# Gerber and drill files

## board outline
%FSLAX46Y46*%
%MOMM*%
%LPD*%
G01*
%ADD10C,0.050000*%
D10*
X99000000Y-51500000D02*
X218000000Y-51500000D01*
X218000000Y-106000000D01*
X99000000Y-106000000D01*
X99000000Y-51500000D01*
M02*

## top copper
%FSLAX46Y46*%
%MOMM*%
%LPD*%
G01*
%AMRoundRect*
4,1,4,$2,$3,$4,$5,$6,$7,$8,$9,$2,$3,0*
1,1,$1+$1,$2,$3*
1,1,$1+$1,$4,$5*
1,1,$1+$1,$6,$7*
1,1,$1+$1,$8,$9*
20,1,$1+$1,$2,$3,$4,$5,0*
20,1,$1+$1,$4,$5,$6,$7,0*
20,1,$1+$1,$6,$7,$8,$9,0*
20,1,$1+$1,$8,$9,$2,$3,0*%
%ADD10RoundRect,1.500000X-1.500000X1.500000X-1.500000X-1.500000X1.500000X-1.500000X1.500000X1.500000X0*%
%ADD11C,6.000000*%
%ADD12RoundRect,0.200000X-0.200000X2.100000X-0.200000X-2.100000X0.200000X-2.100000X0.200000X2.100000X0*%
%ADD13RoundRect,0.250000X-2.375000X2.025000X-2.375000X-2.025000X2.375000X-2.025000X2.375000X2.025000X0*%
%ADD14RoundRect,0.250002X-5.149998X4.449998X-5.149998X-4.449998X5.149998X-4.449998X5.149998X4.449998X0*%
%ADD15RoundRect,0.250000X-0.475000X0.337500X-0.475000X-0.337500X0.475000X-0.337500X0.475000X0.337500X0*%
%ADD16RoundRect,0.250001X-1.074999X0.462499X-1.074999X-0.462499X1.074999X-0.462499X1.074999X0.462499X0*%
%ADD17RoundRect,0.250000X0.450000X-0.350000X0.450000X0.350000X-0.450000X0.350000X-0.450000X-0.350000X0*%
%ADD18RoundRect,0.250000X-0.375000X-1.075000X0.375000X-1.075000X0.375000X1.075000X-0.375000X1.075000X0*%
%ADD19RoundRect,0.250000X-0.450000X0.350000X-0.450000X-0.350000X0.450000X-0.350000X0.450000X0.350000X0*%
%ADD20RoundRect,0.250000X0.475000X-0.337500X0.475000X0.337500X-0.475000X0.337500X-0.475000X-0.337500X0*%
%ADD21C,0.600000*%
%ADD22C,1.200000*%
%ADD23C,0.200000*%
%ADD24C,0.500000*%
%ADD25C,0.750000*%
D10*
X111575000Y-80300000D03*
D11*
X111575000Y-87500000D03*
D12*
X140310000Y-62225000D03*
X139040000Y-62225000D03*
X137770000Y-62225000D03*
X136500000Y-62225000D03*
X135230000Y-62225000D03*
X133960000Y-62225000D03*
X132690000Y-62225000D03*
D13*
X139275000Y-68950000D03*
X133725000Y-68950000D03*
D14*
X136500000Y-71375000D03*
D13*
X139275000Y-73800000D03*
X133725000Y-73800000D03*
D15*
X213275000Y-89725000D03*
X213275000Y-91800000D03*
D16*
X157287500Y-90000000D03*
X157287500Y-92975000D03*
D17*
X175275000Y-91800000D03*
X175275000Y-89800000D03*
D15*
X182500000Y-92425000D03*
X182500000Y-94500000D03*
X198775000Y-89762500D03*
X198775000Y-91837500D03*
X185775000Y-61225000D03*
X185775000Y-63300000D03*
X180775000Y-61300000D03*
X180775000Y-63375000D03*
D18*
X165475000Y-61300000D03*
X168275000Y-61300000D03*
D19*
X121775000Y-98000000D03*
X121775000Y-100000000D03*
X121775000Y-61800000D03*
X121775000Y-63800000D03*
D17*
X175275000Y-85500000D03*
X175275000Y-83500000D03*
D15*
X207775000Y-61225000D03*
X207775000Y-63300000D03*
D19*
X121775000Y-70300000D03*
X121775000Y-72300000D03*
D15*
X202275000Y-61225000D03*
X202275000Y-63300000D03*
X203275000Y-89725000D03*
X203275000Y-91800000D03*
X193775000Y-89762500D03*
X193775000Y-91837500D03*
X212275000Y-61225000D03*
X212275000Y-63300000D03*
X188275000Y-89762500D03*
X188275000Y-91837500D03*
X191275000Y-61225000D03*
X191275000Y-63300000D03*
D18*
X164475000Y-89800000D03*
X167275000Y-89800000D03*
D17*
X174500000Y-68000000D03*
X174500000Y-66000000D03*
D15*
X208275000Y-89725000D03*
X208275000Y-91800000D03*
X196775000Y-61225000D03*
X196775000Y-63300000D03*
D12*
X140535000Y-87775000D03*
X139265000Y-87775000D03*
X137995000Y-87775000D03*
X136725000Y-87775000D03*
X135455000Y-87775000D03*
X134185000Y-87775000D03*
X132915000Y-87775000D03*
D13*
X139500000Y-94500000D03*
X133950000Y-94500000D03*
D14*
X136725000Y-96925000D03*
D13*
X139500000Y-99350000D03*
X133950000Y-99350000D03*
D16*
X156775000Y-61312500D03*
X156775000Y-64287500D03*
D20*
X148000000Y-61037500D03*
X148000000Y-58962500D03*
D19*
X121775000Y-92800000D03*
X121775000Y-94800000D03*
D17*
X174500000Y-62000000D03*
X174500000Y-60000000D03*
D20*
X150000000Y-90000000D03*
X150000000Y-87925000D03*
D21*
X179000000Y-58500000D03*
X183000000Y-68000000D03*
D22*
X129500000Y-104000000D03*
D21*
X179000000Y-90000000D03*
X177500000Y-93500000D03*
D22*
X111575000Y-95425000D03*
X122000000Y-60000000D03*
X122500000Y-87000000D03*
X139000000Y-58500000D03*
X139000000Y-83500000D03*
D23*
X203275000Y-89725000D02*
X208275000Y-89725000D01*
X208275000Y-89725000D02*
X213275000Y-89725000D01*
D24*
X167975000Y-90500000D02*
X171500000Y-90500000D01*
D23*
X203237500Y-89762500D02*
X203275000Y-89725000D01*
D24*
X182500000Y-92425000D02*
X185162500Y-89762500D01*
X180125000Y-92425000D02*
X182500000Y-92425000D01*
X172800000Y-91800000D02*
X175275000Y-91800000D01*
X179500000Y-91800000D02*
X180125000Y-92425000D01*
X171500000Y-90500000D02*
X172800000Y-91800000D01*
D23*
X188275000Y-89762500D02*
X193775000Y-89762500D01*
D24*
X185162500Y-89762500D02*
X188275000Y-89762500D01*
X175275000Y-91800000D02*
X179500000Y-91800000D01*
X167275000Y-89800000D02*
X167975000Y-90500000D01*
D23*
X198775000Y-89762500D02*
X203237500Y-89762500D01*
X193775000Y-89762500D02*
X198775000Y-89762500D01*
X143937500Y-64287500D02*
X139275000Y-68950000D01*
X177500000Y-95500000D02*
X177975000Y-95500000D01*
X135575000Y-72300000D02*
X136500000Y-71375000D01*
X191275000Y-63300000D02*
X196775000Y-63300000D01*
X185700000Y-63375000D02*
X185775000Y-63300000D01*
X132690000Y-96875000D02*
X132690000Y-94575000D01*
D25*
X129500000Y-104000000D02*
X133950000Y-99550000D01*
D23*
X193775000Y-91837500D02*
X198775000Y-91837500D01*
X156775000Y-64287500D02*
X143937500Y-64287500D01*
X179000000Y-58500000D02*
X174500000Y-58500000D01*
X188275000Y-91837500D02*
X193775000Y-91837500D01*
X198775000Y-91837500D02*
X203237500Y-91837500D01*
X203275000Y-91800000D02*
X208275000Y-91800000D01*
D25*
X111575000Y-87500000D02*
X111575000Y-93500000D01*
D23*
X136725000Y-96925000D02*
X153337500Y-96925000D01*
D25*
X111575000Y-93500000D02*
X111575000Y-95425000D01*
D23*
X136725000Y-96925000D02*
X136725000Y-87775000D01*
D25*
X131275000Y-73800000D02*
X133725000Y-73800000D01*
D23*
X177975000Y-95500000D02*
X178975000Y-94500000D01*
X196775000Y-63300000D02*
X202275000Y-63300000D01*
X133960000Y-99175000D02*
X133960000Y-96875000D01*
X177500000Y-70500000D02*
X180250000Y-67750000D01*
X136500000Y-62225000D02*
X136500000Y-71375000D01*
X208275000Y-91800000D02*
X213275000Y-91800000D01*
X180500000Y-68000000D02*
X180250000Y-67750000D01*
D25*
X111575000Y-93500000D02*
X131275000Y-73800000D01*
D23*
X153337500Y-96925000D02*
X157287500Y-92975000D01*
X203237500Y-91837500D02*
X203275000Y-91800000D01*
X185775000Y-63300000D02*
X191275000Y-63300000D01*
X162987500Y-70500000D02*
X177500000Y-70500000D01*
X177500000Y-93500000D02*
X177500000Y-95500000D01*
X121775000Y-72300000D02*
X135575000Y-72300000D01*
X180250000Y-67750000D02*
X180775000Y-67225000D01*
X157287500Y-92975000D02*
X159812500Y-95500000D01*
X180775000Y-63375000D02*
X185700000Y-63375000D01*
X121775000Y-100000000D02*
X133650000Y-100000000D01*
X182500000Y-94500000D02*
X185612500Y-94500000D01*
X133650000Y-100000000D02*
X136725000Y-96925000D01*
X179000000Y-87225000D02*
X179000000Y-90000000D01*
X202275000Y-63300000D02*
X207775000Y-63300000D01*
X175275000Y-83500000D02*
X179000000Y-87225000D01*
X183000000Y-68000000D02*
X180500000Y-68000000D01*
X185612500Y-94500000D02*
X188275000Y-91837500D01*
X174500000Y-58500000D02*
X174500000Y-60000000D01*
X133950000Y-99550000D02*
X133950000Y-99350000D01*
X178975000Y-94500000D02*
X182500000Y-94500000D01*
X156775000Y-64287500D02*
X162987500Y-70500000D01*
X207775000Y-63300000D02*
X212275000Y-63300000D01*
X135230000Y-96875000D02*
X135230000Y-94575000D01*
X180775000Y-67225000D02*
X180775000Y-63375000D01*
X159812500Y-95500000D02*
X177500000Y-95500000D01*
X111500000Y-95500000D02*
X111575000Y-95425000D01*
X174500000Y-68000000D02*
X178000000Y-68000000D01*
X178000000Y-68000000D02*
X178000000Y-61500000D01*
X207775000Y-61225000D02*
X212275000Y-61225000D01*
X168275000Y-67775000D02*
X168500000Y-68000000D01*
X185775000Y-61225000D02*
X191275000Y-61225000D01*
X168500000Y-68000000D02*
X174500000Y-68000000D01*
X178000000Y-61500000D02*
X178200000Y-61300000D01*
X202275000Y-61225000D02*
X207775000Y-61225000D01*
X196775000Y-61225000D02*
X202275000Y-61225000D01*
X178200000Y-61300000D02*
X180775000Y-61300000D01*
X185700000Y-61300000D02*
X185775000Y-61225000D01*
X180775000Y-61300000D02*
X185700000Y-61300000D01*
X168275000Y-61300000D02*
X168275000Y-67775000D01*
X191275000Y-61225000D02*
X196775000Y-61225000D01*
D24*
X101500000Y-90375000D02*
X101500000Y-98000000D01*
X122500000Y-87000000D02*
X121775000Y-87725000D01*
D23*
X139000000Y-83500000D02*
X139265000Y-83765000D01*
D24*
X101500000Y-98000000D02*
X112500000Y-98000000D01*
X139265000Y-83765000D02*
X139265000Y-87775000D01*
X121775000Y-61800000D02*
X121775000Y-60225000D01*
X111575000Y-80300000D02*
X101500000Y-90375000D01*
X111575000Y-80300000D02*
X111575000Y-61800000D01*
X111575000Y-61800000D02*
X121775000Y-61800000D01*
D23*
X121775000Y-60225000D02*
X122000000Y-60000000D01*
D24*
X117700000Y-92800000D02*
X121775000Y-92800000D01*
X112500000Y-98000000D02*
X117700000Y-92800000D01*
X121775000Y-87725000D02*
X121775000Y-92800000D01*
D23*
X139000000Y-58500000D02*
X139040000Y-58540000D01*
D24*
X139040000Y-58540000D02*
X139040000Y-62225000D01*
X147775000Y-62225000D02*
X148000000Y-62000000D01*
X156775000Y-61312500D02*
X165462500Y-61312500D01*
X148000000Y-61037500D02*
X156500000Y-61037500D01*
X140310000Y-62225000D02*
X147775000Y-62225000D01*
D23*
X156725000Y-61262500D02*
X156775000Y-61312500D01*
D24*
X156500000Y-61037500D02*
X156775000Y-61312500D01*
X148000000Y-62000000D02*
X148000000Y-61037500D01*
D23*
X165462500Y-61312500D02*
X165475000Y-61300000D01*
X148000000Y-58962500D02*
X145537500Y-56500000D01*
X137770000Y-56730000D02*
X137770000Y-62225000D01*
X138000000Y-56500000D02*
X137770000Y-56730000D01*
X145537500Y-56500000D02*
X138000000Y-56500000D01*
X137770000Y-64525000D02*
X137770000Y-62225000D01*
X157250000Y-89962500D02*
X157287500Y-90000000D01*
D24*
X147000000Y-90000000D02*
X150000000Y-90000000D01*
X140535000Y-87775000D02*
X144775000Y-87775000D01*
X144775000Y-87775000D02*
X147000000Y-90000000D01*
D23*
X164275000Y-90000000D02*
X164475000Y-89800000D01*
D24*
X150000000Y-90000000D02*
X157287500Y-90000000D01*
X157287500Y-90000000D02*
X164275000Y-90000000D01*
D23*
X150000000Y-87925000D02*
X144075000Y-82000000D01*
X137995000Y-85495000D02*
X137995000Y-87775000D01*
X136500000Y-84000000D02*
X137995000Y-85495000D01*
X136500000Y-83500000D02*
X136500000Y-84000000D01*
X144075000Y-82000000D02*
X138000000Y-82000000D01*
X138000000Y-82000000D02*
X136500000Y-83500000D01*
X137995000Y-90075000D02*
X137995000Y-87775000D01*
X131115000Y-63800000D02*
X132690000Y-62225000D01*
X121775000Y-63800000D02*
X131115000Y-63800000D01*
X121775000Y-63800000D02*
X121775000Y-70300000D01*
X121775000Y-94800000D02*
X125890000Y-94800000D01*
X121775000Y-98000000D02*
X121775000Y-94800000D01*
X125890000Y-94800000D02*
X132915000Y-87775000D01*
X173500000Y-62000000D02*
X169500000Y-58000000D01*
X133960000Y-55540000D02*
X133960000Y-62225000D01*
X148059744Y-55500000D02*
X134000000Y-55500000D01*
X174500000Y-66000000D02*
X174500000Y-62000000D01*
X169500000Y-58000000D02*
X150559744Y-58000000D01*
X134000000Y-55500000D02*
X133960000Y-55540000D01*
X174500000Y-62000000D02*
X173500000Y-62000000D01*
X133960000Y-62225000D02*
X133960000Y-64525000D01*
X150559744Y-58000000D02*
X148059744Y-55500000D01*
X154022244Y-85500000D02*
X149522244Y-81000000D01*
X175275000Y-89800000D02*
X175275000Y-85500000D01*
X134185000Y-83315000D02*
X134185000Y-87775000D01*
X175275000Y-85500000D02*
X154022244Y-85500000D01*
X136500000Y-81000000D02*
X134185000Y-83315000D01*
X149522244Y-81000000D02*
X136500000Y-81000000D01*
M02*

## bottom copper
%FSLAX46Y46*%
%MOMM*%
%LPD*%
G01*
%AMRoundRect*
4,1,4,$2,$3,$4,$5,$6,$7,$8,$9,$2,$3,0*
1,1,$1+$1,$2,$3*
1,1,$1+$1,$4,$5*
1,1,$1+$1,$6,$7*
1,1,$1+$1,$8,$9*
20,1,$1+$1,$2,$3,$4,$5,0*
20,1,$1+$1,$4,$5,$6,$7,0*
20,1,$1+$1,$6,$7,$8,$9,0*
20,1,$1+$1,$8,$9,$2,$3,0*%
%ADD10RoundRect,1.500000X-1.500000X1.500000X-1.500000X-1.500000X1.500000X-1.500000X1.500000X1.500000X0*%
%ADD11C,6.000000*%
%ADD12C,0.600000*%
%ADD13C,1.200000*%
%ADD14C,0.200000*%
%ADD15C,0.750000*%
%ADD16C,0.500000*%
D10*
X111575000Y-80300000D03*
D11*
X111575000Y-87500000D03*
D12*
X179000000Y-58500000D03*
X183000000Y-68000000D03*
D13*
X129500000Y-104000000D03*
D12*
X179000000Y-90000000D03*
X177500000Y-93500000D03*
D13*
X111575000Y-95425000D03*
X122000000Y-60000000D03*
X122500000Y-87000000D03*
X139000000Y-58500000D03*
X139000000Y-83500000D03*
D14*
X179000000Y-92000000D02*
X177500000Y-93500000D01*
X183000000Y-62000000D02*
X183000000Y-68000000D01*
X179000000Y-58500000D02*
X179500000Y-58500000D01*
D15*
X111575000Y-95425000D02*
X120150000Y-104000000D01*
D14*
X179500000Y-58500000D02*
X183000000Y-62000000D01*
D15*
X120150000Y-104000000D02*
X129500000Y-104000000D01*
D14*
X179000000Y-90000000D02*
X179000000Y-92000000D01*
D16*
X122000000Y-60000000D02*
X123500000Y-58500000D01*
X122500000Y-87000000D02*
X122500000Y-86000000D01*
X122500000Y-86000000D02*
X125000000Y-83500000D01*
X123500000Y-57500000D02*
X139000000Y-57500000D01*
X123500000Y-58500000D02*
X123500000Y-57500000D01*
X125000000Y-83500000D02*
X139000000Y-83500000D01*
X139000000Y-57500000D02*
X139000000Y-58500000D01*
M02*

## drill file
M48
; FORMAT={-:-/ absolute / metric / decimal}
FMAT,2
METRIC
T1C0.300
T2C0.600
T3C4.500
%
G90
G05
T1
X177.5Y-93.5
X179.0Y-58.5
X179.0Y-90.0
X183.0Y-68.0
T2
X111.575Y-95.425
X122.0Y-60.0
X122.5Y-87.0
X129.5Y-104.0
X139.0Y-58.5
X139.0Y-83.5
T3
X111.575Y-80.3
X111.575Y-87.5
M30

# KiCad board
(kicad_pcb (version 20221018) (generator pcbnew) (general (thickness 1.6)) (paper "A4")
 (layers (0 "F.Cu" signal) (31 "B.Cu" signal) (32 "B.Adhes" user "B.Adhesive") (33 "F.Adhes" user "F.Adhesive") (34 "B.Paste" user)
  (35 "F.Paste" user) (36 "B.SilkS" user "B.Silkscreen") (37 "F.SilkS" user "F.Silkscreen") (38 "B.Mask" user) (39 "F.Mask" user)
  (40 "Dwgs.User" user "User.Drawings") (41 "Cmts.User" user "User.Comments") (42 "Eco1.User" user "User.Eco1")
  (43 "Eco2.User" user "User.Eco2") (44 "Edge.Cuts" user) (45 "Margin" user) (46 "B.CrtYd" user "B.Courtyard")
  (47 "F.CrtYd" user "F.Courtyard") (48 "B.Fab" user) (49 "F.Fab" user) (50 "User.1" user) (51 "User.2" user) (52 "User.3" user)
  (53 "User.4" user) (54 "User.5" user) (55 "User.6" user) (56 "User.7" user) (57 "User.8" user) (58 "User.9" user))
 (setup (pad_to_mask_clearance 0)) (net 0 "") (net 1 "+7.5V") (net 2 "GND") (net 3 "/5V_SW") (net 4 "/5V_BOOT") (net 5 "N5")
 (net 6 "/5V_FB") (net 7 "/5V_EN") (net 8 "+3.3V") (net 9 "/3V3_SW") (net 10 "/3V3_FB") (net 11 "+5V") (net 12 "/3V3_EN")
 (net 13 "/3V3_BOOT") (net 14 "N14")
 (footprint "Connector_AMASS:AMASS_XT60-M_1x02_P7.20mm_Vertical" (layer "F.Cu") (at 111.575 80.3 -90)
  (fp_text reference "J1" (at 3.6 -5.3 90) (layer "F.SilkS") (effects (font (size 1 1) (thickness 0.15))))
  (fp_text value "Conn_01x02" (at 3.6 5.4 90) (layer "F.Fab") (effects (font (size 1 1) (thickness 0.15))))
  (pad "1" thru_hole roundrect (at 0 0 270) (size 6 6) (drill 4.5) (layers "*.Cu" "*.Mask") (roundrect_rratio 0.25) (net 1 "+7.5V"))
  (pad "2" thru_hole circle (at 7.2 0 270) (size 6 6) (drill 4.5) (layers "*.Cu" "*.Mask") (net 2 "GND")))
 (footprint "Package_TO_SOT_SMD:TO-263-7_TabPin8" (layer "F.Cu") (at 136.5 69.875 -90)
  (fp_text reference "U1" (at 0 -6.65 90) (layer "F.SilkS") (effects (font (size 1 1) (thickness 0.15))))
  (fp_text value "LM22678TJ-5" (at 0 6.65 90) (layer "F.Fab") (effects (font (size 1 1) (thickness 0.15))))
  (pad "1" smd roundrect (at -7.65 -3.81 270) (size 4.6 0.8) (layers "F.Cu" "F.Paste" "F.Mask") (roundrect_rratio 0.25) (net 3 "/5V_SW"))
  (pad "2" smd roundrect (at -7.65 -2.54 270) (size 4.6 0.8) (layers "F.Cu" "F.Paste" "F.Mask") (roundrect_rratio 0.25) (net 1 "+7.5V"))
  (pad "3" smd roundrect (at -7.65 -1.27 270) (size 4.6 0.8) (layers "F.Cu" "F.Paste" "F.Mask") (roundrect_rratio 0.25) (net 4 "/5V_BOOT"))
  (pad "4" smd roundrect (at -7.65 0 270) (size 4.6 0.8) (layers "F.Cu" "F.Paste" "F.Mask") (roundrect_rratio 0.25) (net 2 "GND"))
  (pad "5" smd roundrect (at -7.65 1.27 270) (size 4.6 0.8) (layers "F.Cu" "F.Paste" "F.Mask") (roundrect_rratio 0.25) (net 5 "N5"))
  (pad "6" smd roundrect (at -7.65 2.54 270) (size 4.6 0.8) (layers "F.Cu" "F.Paste" "F.Mask") (roundrect_rratio 0.25) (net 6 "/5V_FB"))
  (pad "7" smd roundrect (at -7.65 3.81 270) (size 4.6 0.8) (layers "F.Cu" "F.Paste" "F.Mask") (roundrect_rratio 0.25) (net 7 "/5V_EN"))
  (pad "8" smd roundrect (at -0.925 -2.775 270) (size 4.55 5.25) (layers "F.Cu" "F.Paste") (roundrect_rratio 0.054945) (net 2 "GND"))
  (pad "8" smd roundrect (at -0.925 2.775 270) (size 4.55 5.25) (layers "F.Cu" "F.Paste") (roundrect_rratio 0.054945) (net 2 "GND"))
  (pad "8" smd roundrect (at 1.5 0 270) (size 9.4 10.8) (layers "F.Cu" "F.Mask") (roundrect_rratio 0.026596) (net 2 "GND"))
  (pad "8" smd roundrect (at 3.925 -2.775 270) (size 4.55 5.25) (layers "F.Cu" "F.Paste") (roundrect_rratio 0.054945) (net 2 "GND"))
  (pad "8" smd roundrect (at 3.925 2.775 270) (size 4.55 5.25) (layers "F.Cu" "F.Paste") (roundrect_rratio 0.054945) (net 2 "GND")))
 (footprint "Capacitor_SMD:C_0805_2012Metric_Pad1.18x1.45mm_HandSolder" (layer "F.Cu") (at 213.275 90.7625 -90)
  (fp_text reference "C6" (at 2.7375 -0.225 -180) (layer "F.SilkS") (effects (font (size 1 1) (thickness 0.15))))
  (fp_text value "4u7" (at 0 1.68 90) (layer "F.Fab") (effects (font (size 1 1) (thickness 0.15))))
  (pad "1" smd roundrect (at -1.0375 0 270) (size 1.175 1.45) (layers "F.Cu" "F.Paste" "F.Mask") (roundrect_rratio 0.212766) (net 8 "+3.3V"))
  (pad "2" smd roundrect (at 1.0375 0 270) (size 1.175 1.45) (layers "F.Cu" "F.Paste" "F.Mask") (roundrect_rratio 0.212766) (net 2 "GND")))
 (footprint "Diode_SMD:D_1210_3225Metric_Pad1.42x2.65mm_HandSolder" (layer "F.Cu") (at 157.2875 91.4875 -90)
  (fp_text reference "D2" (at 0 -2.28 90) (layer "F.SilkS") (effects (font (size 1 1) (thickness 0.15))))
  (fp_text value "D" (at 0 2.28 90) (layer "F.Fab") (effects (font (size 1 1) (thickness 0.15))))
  (pad "1" smd roundrect (at -1.4875 0 270) (size 1.425 2.65) (layers "F.Cu" "F.Paste" "F.Mask") (roundrect_rratio 0.175439)
   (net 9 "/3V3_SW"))
  (pad "2" smd roundrect (at 1.4875 0 270) (size 1.425 2.65) (layers "F.Cu" "F.Paste" "F.Mask") (roundrect_rratio 0.175439) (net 2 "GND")))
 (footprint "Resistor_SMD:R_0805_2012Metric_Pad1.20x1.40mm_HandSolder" (layer "F.Cu") (at 175.275 90.8 90)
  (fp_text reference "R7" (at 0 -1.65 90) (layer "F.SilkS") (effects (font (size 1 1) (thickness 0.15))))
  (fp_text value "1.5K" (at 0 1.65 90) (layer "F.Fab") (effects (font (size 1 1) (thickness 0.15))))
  (pad "1" smd roundrect (at -1 0 90) (size 1.2 1.4) (layers "F.Cu" "F.Paste" "F.Mask") (roundrect_rratio 0.208333) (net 8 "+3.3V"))
  (pad "2" smd roundrect (at 1 0 90) (size 1.2 1.4) (layers "F.Cu" "F.Paste" "F.Mask") (roundrect_rratio 0.208333) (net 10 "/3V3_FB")))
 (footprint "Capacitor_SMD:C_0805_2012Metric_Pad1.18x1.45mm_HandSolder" (layer "F.Cu") (at 182.5 93.4625 -90)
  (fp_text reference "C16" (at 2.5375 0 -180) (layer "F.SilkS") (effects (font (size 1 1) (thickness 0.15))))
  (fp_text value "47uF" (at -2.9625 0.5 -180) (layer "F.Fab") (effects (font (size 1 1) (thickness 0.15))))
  (pad "1" smd roundrect (at -1.0375 0 270) (size 1.175 1.45) (layers "F.Cu" "F.Paste" "F.Mask") (roundrect_rratio 0.212766) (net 8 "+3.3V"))
  (pad "2" smd roundrect (at 1.0375 0 270) (size 1.175 1.45) (layers "F.Cu" "F.Paste" "F.Mask") (roundrect_rratio 0.212766) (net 2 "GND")))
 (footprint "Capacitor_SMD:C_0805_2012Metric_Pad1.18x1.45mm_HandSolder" (layer "F.Cu") (at 198.775 90.8 -90)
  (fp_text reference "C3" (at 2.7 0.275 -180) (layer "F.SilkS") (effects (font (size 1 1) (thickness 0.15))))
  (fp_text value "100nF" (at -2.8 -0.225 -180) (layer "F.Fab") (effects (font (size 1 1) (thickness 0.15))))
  (pad "1" smd roundrect (at -1.0375 0 270) (size 1.175 1.45) (layers "F.Cu" "F.Paste" "F.Mask") (roundrect_rratio 0.212766) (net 8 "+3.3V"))
  (pad "2" smd roundrect (at 1.0375 0 270) (size 1.175 1.45) (layers "F.Cu" "F.Paste" "F.Mask") (roundrect_rratio 0.212766) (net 2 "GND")))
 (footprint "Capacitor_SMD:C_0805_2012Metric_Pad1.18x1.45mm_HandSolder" (layer "F.Cu") (at 185.775 62.2625 -90)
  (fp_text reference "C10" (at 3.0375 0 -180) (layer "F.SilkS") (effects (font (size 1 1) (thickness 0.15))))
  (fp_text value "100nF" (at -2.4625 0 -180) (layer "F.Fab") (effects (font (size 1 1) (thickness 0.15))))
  (pad "1" smd roundrect (at -1.0375 0 270) (size 1.175 1.45) (layers "F.Cu" "F.Paste" "F.Mask") (roundrect_rratio 0.212766) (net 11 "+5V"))
  (pad "2" smd roundrect (at 1.0375 0 270) (size 1.175 1.45) (layers "F.Cu" "F.Paste" "F.Mask") (roundrect_rratio 0.212766) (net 2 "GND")))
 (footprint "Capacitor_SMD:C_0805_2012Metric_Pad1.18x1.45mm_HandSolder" (layer "F.Cu") (at 180.775 62.3375 -90)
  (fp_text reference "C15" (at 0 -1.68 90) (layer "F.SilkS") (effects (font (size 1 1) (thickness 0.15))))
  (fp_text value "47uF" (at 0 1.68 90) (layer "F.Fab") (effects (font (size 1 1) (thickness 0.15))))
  (pad "1" smd roundrect (at -1.0375 0 270) (size 1.175 1.45) (layers "F.Cu" "F.Paste" "F.Mask") (roundrect_rratio 0.212766) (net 11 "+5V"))
  (pad "2" smd roundrect (at 1.0375 0 270) (size 1.175 1.45) (layers "F.Cu" "F.Paste" "F.Mask") (roundrect_rratio 0.212766) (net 2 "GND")))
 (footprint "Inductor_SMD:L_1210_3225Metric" (layer "F.Cu") (at 166.875 61.3)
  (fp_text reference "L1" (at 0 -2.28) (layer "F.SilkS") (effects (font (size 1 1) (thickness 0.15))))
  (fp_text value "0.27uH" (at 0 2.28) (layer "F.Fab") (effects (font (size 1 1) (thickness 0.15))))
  (pad "1" smd roundrect (at -1.4 0) (size 1.25 2.65) (layers "F.Cu" "F.Paste" "F.Mask") (roundrect_rratio 0.2) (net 3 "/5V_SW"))
  (pad "2" smd roundrect (at 1.4 0) (size 1.25 2.65) (layers "F.Cu" "F.Paste" "F.Mask") (roundrect_rratio 0.2) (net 11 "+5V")))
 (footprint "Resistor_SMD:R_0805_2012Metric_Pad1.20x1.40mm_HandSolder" (layer "F.Cu") (at 121.775 99 -90)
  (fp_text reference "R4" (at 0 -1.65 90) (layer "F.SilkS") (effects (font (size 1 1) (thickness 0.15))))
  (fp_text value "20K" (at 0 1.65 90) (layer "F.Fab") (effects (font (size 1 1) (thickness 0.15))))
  (pad "1" smd roundrect (at -1 0 270) (size 1.2 1.4) (layers "F.Cu" "F.Paste" "F.Mask") (roundrect_rratio 0.208333) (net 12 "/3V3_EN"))
  (pad "2" smd roundrect (at 1 0 270) (size 1.2 1.4) (layers "F.Cu" "F.Paste" "F.Mask") (roundrect_rratio 0.208333) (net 2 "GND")))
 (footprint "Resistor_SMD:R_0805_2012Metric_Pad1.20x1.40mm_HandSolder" (layer "F.Cu") (at 121.775 62.8 -90)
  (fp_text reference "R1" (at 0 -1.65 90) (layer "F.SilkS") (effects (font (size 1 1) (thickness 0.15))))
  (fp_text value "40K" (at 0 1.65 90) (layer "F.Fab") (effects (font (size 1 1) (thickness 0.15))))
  (pad "1" smd roundrect (at -1 0 270) (size 1.2 1.4) (layers "F.Cu" "F.Paste" "F.Mask") (roundrect_rratio 0.208333) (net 1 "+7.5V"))
  (pad "2" smd roundrect (at 1 0 270) (size 1.2 1.4) (layers "F.Cu" "F.Paste" "F.Mask") (roundrect_rratio 0.208333) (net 7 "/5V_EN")))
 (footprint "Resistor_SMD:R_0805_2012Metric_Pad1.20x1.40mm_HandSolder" (layer "F.Cu") (at 175.275 84.5 90)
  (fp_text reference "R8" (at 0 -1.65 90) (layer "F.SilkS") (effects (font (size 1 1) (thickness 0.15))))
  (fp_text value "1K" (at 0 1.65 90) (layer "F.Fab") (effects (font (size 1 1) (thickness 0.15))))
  (pad "1" smd roundrect (at -1 0 90) (size 1.2 1.4) (layers "F.Cu" "F.Paste" "F.Mask") (roundrect_rratio 0.208333) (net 10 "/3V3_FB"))
  (pad "2" smd roundrect (at 1 0 90) (size 1.2 1.4) (layers "F.Cu" "F.Paste" "F.Mask") (roundrect_rratio 0.208333) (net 2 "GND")))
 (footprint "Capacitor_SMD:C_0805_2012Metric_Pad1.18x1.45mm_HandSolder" (layer "F.Cu") (at 207.775 62.2625 -90)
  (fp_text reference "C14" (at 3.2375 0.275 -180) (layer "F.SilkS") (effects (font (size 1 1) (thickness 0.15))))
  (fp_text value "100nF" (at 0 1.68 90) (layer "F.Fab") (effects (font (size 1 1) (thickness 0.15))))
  (pad "1" smd roundrect (at -1.0375 0 270) (size 1.175 1.45) (layers "F.Cu" "F.Paste" "F.Mask") (roundrect_rratio 0.212766) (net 11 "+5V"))
  (pad "2" smd roundrect (at 1.0375 0 270) (size 1.175 1.45) (layers "F.Cu" "F.Paste" "F.Mask") (roundrect_rratio 0.212766) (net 2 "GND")))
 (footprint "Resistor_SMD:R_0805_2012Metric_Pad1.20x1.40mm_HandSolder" (layer "F.Cu") (at 121.775 71.3 -90)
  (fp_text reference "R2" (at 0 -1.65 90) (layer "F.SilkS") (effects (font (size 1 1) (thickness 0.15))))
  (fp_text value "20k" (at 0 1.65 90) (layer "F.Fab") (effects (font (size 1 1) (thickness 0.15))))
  (pad "1" smd roundrect (at -1 0 270) (size 1.2 1.4) (layers "F.Cu" "F.Paste" "F.Mask") (roundrect_rratio 0.208333) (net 7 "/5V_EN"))
  (pad "2" smd roundrect (at 1 0 270) (size 1.2 1.4) (layers "F.Cu" "F.Paste" "F.Mask") (roundrect_rratio 0.208333) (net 2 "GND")))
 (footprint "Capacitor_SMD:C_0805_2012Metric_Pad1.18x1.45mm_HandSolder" (layer "F.Cu") (at 202.275 62.2625 -90)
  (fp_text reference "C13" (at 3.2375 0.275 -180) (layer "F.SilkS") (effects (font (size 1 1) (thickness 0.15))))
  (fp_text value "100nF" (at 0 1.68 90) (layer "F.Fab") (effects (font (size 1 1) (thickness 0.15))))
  (pad "1" smd roundrect (at -1.0375 0 270) (size 1.175 1.45) (layers "F.Cu" "F.Paste" "F.Mask") (roundrect_rratio 0.212766) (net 11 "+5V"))
  (pad "2" smd roundrect (at 1.0375 0 270) (size 1.175 1.45) (layers "F.Cu" "F.Paste" "F.Mask") (roundrect_rratio 0.212766) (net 2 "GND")))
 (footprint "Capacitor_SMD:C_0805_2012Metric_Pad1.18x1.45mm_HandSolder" (layer "F.Cu") (at 203.275 90.7625 -90)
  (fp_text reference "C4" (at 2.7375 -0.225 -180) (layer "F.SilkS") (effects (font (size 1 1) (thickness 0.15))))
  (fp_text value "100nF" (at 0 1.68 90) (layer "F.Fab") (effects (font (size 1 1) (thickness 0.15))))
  (pad "1" smd roundrect (at -1.0375 0 270) (size 1.175 1.45) (layers "F.Cu" "F.Paste" "F.Mask") (roundrect_rratio 0.212766) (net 8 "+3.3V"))
  (pad "2" smd roundrect (at 1.0375 0 270) (size 1.175 1.45) (layers "F.Cu" "F.Paste" "F.Mask") (roundrect_rratio 0.212766) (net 2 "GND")))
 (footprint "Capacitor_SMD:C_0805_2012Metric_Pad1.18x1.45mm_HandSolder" (layer "F.Cu") (at 193.775 90.8 -90)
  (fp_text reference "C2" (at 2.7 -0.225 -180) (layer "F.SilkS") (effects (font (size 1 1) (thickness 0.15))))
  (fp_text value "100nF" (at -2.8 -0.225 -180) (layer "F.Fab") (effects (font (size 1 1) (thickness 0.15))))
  (pad "1" smd roundrect (at -1.0375 0 270) (size 1.175 1.45) (layers "F.Cu" "F.Paste" "F.Mask") (roundrect_rratio 0.212766) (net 8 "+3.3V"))
  (pad "2" smd roundrect (at 1.0375 0 270) (size 1.175 1.45) (layers "F.Cu" "F.Paste" "F.Mask") (roundrect_rratio 0.212766) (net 2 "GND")))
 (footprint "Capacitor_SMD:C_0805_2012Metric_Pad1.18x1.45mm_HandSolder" (layer "F.Cu") (at 212.275 62.2625 -90)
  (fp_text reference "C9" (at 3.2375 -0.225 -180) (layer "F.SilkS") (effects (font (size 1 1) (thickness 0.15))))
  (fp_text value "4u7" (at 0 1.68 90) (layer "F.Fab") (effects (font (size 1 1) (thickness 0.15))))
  (pad "1" smd roundrect (at -1.0375 0 270) (size 1.175 1.45) (layers "F.Cu" "F.Paste" "F.Mask") (roundrect_rratio 0.212766) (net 11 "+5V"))
  (pad "2" smd roundrect (at 1.0375 0 270) (size 1.175 1.45) (layers "F.Cu" "F.Paste" "F.Mask") (roundrect_rratio 0.212766) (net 2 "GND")))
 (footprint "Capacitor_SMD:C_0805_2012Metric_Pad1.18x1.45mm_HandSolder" (layer "F.Cu") (at 188.275 90.8 -90)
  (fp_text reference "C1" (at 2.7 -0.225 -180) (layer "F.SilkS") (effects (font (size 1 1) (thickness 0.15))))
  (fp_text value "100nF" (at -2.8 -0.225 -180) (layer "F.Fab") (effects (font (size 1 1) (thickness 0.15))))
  (pad "1" smd roundrect (at -1.0375 0 270) (size 1.175 1.45) (layers "F.Cu" "F.Paste" "F.Mask") (roundrect_rratio 0.212766) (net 8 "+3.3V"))
  (pad "2" smd roundrect (at 1.0375 0 270) (size 1.175 1.45) (layers "F.Cu" "F.Paste" "F.Mask") (roundrect_rratio 0.212766) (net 2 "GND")))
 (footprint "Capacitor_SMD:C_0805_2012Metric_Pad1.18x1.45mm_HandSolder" (layer "F.Cu") (at 191.275 62.2625 -90)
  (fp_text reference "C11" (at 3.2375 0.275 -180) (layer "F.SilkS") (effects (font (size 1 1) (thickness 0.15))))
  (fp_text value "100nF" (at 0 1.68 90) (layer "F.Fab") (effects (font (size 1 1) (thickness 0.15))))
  (pad "1" smd roundrect (at -1.0375 0 270) (size 1.175 1.45) (layers "F.Cu" "F.Paste" "F.Mask") (roundrect_rratio 0.212766) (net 11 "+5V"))
  (pad "2" smd roundrect (at 1.0375 0 270) (size 1.175 1.45) (layers "F.Cu" "F.Paste" "F.Mask") (roundrect_rratio 0.212766) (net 2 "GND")))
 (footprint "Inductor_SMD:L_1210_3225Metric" (layer "F.Cu") (at 165.875 89.8)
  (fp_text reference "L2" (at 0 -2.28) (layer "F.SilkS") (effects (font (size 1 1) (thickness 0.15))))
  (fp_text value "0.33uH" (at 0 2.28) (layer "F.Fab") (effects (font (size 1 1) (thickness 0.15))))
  (pad "1" smd roundrect (at -1.4 0) (size 1.25 2.65) (layers "F.Cu" "F.Paste" "F.Mask") (roundrect_rratio 0.2) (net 9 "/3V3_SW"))
  (pad "2" smd roundrect (at 1.4 0) (size 1.25 2.65) (layers "F.Cu" "F.Paste" "F.Mask") (roundrect_rratio 0.2) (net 8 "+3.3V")))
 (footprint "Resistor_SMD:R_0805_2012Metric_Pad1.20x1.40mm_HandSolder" (layer "F.Cu") (at 174.5 67 90)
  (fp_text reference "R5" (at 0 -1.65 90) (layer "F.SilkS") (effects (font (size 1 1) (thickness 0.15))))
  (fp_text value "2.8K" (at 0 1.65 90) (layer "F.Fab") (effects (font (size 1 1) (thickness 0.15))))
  (pad "1" smd roundrect (at -1 0 90) (size 1.2 1.4) (layers "F.Cu" "F.Paste" "F.Mask") (roundrect_rratio 0.208333) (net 11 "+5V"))
  (pad "2" smd roundrect (at 1 0 90) (size 1.2 1.4) (layers "F.Cu" "F.Paste" "F.Mask") (roundrect_rratio 0.208333) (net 6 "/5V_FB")))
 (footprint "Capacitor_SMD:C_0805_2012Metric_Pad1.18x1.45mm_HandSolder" (layer "F.Cu") (at 208.275 90.7625 -90)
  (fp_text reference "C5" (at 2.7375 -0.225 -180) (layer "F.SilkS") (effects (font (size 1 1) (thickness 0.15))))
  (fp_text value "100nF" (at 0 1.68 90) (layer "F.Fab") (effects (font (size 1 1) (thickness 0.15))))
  (pad "1" smd roundrect (at -1.0375 0 270) (size 1.175 1.45) (layers "F.Cu" "F.Paste" "F.Mask") (roundrect_rratio 0.212766) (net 8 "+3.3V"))
  (pad "2" smd roundrect (at 1.0375 0 270) (size 1.175 1.45) (layers "F.Cu" "F.Paste" "F.Mask") (roundrect_rratio 0.212766) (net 2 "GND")))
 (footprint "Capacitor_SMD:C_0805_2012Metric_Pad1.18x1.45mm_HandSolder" (layer "F.Cu") (at 196.775 62.2625 -90)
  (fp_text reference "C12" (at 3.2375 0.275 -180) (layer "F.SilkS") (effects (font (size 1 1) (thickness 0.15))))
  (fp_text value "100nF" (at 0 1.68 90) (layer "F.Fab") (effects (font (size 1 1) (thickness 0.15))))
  (pad "1" smd roundrect (at -1.0375 0 270) (size 1.175 1.45) (layers "F.Cu" "F.Paste" "F.Mask") (roundrect_rratio 0.212766) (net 11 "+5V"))
  (pad "2" smd roundrect (at 1.0375 0 270) (size 1.175 1.45) (layers "F.Cu" "F.Paste" "F.Mask") (roundrect_rratio 0.212766) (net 2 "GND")))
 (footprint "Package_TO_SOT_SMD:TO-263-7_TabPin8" (layer "F.Cu") (at 136.725 95.425 -90)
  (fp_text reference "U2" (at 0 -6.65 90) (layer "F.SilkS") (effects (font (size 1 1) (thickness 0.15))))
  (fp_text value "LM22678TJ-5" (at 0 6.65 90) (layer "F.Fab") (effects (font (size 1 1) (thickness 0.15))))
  (pad "1" smd roundrect (at -7.65 -3.81 270) (size 4.6 0.8) (layers "F.Cu" "F.Paste" "F.Mask") (roundrect_rratio 0.25) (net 9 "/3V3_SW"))
  (pad "2" smd roundrect (at -7.65 -2.54 270) (size 4.6 0.8) (layers "F.Cu" "F.Paste" "F.Mask") (roundrect_rratio 0.25) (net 1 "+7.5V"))
  (pad "3" smd roundrect (at -7.65 -1.27 270) (size 4.6 0.8) (layers "F.Cu" "F.Paste" "F.Mask") (roundrect_rratio 0.25) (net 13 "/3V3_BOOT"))
  (pad "4" smd roundrect (at -7.65 0 270) (size 4.6 0.8) (layers "F.Cu" "F.Paste" "F.Mask") (roundrect_rratio 0.25) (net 2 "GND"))
  (pad "5" smd roundrect (at -7.65 1.27 270) (size 4.6 0.8) (layers "F.Cu" "F.Paste" "F.Mask") (roundrect_rratio 0.25) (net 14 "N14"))
  (pad "6" smd roundrect (at -7.65 2.54 270) (size 4.6 0.8) (layers "F.Cu" "F.Paste" "F.Mask") (roundrect_rratio 0.25) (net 10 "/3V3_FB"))
  (pad "7" smd roundrect (at -7.65 3.81 270) (size 4.6 0.8) (layers "F.Cu" "F.Paste" "F.Mask") (roundrect_rratio 0.25) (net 12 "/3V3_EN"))
  (pad "8" smd roundrect (at -0.925 -2.775 270) (size 4.55 5.25) (layers "F.Cu" "F.Paste") (roundrect_rratio 0.054945) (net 2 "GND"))
  (pad "8" smd roundrect (at -0.925 2.775 270) (size 4.55 5.25) (layers "F.Cu" "F.Paste") (roundrect_rratio 0.054945) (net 2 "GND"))
  (pad "8" smd roundrect (at 1.5 0 270) (size 9.4 10.8) (layers "F.Cu" "F.Mask") (roundrect_rratio 0.026596) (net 2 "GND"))
  (pad "8" smd roundrect (at 3.925 -2.775 270) (size 4.55 5.25) (layers "F.Cu" "F.Paste") (roundrect_rratio 0.054945) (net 2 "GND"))
  (pad "8" smd roundrect (at 3.925 2.775 270) (size 4.55 5.25) (layers "F.Cu" "F.Paste") (roundrect_rratio 0.054945) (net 2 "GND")))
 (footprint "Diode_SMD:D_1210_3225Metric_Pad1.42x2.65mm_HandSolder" (layer "F.Cu") (at 156.775 62.8 -90)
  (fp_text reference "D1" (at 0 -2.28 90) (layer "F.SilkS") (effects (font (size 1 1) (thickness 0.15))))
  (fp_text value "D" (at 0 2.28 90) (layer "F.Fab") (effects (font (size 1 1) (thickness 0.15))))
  (pad "1" smd roundrect (at -1.4875 0 270) (size 1.425 2.65) (layers "F.Cu" "F.Paste" "F.Mask") (roundrect_rratio 0.175439)
   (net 3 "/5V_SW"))
  (pad "2" smd roundrect (at 1.4875 0 270) (size 1.425 2.65) (layers "F.Cu" "F.Paste" "F.Mask") (roundrect_rratio 0.175439) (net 2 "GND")))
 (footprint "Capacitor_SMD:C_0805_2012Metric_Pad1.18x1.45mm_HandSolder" (layer "F.Cu") (at 148 60 90)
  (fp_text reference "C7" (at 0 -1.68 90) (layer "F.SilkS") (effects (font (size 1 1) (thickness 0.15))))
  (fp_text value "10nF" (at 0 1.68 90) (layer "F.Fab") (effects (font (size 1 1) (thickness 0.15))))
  (pad "1" smd roundrect (at -1.0375 0 90) (size 1.175 1.45) (layers "F.Cu" "F.Paste" "F.Mask") (roundrect_rratio 0.212766) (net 3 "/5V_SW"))
  (pad "2" smd roundrect (at 1.0375 0 90) (size 1.175 1.45) (layers "F.Cu" "F.Paste" "F.Mask") (roundrect_rratio 0.212766)
   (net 4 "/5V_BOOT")))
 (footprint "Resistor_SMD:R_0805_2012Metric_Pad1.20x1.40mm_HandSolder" (layer "F.Cu") (at 121.775 93.8 -90)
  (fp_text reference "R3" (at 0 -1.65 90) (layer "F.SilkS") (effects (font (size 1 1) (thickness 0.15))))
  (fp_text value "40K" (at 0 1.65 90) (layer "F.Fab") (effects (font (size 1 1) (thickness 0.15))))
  (pad "1" smd roundrect (at -1 0 270) (size 1.2 1.4) (layers "F.Cu" "F.Paste" "F.Mask") (roundrect_rratio 0.208333) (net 1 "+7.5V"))
  (pad "2" smd roundrect (at 1 0 270) (size 1.2 1.4) (layers "F.Cu" "F.Paste" "F.Mask") (roundrect_rratio 0.208333) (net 12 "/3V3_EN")))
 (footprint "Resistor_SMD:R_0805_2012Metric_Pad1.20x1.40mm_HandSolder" (layer "F.Cu") (at 174.5 61 90)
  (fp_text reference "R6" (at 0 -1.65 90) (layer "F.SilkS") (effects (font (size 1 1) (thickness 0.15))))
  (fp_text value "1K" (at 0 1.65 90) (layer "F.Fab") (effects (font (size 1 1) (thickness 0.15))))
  (pad "1" smd roundrect (at -1 0 90) (size 1.2 1.4) (layers "F.Cu" "F.Paste" "F.Mask") (roundrect_rratio 0.208333) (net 6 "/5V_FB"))
  (pad "2" smd roundrect (at 1 0 90) (size 1.2 1.4) (layers "F.Cu" "F.Paste" "F.Mask") (roundrect_rratio 0.208333) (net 2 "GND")))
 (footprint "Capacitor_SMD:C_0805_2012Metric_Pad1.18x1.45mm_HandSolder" (layer "F.Cu") (at 150 88.9625 90)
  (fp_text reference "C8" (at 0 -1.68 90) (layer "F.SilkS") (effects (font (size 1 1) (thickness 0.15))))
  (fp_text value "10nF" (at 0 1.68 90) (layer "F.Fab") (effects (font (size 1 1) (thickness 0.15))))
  (pad "1" smd roundrect (at -1.0375 0 90) (size 1.175 1.45) (layers "F.Cu" "F.Paste" "F.Mask") (roundrect_rratio 0.212766)
   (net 9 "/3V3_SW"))
  (pad "2" smd roundrect (at 1.0375 0 90) (size 1.175 1.45) (layers "F.Cu" "F.Paste" "F.Mask") (roundrect_rratio 0.212766)
   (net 13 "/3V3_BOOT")))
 (gr_rect (start 99 51.5) (end 218 106) (stroke (width 0.05) (type default)) (fill none) (layer "Edge.Cuts"))
 (segment (start 203.275 89.725) (end 208.275 89.725) (width 0.2) (layer "F.Cu") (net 8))
 (segment (start 208.275 89.725) (end 213.275 89.725) (width 0.2) (layer "F.Cu") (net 8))
 (segment (start 167.975 90.5) (end 171.5 90.5) (width 0.5) (layer "F.Cu") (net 8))
 (segment (start 203.2375 89.7625) (end 203.275 89.725) (width 0.2) (layer "F.Cu") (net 8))
 (segment (start 182.5 92.425) (end 185.1625 89.7625) (width 0.5) (layer "F.Cu") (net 8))
 (segment (start 180.125 92.425) (end 182.5 92.425) (width 0.5) (layer "F.Cu") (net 8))
 (segment (start 172.8 91.8) (end 175.275 91.8) (width 0.5) (layer "F.Cu") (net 8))
 (segment (start 179.5 91.8) (end 180.125 92.425) (width 0.5) (layer "F.Cu") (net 8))
 (segment (start 171.5 90.5) (end 172.8 91.8) (width 0.5) (layer "F.Cu") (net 8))
 (segment (start 188.275 89.7625) (end 193.775 89.7625) (width 0.2) (layer "F.Cu") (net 8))
 (segment (start 185.1625 89.7625) (end 188.275 89.7625) (width 0.5) (layer "F.Cu") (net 8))
 (segment (start 175.275 91.8) (end 179.5 91.8) (width 0.5) (layer "F.Cu") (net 8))
 (segment (start 167.275 89.8) (end 167.975 90.5) (width 0.5) (layer "F.Cu") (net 8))
 (segment (start 198.775 89.7625) (end 203.2375 89.7625) (width 0.2) (layer "F.Cu") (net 8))
 (segment (start 193.775 89.7625) (end 198.775 89.7625) (width 0.2) (layer "F.Cu") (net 8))
 (segment (start 143.9375 64.2875) (end 139.275 68.95) (width 0.2) (layer "F.Cu") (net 2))
 (segment (start 177.5 95.5) (end 177.975 95.5) (width 0.2) (layer "F.Cu") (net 2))
 (segment (start 135.575 72.3) (end 136.5 71.375) (width 0.2) (layer "F.Cu") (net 2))
 (segment (start 191.275 63.3) (end 196.775 63.3) (width 0.2) (layer "F.Cu") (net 2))
 (segment (start 185.7 63.375) (end 185.775 63.3) (width 0.2) (layer "F.Cu") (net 2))
 (segment (start 132.69 96.875) (end 132.69 94.575) (width 0.2) (layer "F.Cu") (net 2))
 (segment (start 129.5 104) (end 133.95 99.55) (width 0.75) (layer "F.Cu") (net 2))
 (segment (start 193.775 91.8375) (end 198.775 91.8375) (width 0.2) (layer "F.Cu") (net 2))
 (segment (start 156.775 64.2875) (end 143.9375 64.2875) (width 0.2) (layer "F.Cu") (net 2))
 (segment (start 179 58.5) (end 174.5 58.5) (width 0.2) (layer "F.Cu") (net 2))
 (segment (start 188.275 91.8375) (end 193.775 91.8375) (width 0.2) (layer "F.Cu") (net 2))
 (segment (start 198.775 91.8375) (end 203.2375 91.8375) (width 0.2) (layer "F.Cu") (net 2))
 (segment (start 203.275 91.8) (end 208.275 91.8) (width 0.2) (layer "F.Cu") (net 2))
 (segment (start 111.575 87.5) (end 111.575 93.5) (width 0.75) (layer "F.Cu") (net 2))
 (segment (start 136.725 96.925) (end 153.3375 96.925) (width 0.2) (layer "F.Cu") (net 2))
 (segment (start 111.575 93.5) (end 111.575 95.425) (width 0.75) (layer "F.Cu") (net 2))
 (segment (start 136.725 96.925) (end 136.725 87.775) (width 0.2) (layer "F.Cu") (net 2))
 (segment (start 131.275 73.8) (end 133.725 73.8) (width 0.75) (layer "F.Cu") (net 2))
 (segment (start 177.975 95.5) (end 178.975 94.5) (width 0.2) (layer "F.Cu") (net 2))
 (segment (start 196.775 63.3) (end 202.275 63.3) (width 0.2) (layer "F.Cu") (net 2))
 (segment (start 133.96 99.175) (end 133.96 96.875) (width 0.2) (layer "F.Cu") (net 2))
 (segment (start 177.5 70.5) (end 180.25 67.75) (width 0.2) (layer "F.Cu") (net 2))
 (segment (start 136.5 62.225) (end 136.5 71.375) (width 0.2) (layer "F.Cu") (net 2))
 (segment (start 208.275 91.8) (end 213.275 91.8) (width 0.2) (layer "F.Cu") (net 2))
 (segment (start 180.5 68) (end 180.25 67.75) (width 0.2) (layer "F.Cu") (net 2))
 (segment (start 111.575 93.5) (end 131.275 73.8) (width 0.75) (layer "F.Cu") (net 2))
 (segment (start 153.3375 96.925) (end 157.2875 92.975) (width 0.2) (layer "F.Cu") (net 2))
 (segment (start 203.2375 91.8375) (end 203.275 91.8) (width 0.2) (layer "F.Cu") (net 2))
 (segment (start 185.775 63.3) (end 191.275 63.3) (width 0.2) (layer "F.Cu") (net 2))
 (segment (start 162.9875 70.5) (end 177.5 70.5) (width 0.2) (layer "F.Cu") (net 2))
 (segment (start 177.5 93.5) (end 177.5 95.5) (width 0.2) (layer "F.Cu") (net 2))
 (segment (start 121.775 72.3) (end 135.575 72.3) (width 0.2) (layer "F.Cu") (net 2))
 (segment (start 180.25 67.75) (end 180.775 67.225) (width 0.2) (layer "F.Cu") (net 2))
 (segment (start 157.2875 92.975) (end 159.8125 95.5) (width 0.2) (layer "F.Cu") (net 2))
 (segment (start 180.775 63.375) (end 185.7 63.375) (width 0.2) (layer "F.Cu") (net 2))
 (segment (start 121.775 100) (end 133.65 100) (width 0.2) (layer "F.Cu") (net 2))
 (segment (start 182.5 94.5) (end 185.6125 94.5) (width 0.2) (layer "F.Cu") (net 2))
 (segment (start 133.65 100) (end 136.725 96.925) (width 0.2) (layer "F.Cu") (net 2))
 (segment (start 179 87.225) (end 179 90) (width 0.2) (layer "F.Cu") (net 2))
 (segment (start 202.275 63.3) (end 207.775 63.3) (width 0.2) (layer "F.Cu") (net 2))
 (segment (start 175.275 83.5) (end 179 87.225) (width 0.2) (layer "F.Cu") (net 2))
 (segment (start 183 68) (end 180.5 68) (width 0.2) (layer "F.Cu") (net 2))
 (segment (start 185.6125 94.5) (end 188.275 91.8375) (width 0.2) (layer "F.Cu") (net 2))
 (segment (start 174.5 58.5) (end 174.5 60) (width 0.2) (layer "F.Cu") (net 2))
 (segment (start 133.95 99.55) (end 133.95 99.35) (width 0.2) (layer "F.Cu") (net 2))
 (segment (start 178.975 94.5) (end 182.5 94.5) (width 0.2) (layer "F.Cu") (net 2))
 (segment (start 156.775 64.2875) (end 162.9875 70.5) (width 0.2) (layer "F.Cu") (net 2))
 (segment (start 207.775 63.3) (end 212.275 63.3) (width 0.2) (layer "F.Cu") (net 2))
 (segment (start 135.23 96.875) (end 135.23 94.575) (width 0.2) (layer "F.Cu") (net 2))
 (segment (start 180.775 67.225) (end 180.775 63.375) (width 0.2) (layer "F.Cu") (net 2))
 (segment (start 159.8125 95.5) (end 177.5 95.5) (width 0.2) (layer "F.Cu") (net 2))
 (segment (start 111.5 95.5) (end 111.575 95.425) (width 0.2) (layer "F.Cu") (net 2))
 (via (at 179 58.5) (size 0.6) (drill 0.3) (layers "F.Cu" "B.Cu") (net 2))
 (via (at 183 68) (size 0.6) (drill 0.3) (layers "F.Cu" "B.Cu") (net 2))
 (via (at 129.5 104) (size 1.2) (drill 0.6) (layers "F.Cu" "B.Cu") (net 2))
 (via (at 179 90) (size 0.6) (drill 0.3) (layers "F.Cu" "B.Cu") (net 2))
 (via (at 177.5 93.5) (size 0.6) (drill 0.3) (layers "F.Cu" "B.Cu") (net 2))
 (via (at 111.575 95.425) (size 1.2) (drill 0.6) (layers "F.Cu" "B.Cu") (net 2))
 (segment (start 179 92) (end 177.5 93.5) (width 0.2) (layer "B.Cu") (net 2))
 (segment (start 183 62) (end 183 68) (width 0.2) (layer "B.Cu") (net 2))
 (segment (start 179 58.5) (end 179.5 58.5) (width 0.2) (layer "B.Cu") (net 2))
 (segment (start 111.575 95.425) (end 120.15 104) (width 0.75) (layer "B.Cu") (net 2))
 (segment (start 179.5 58.5) (end 183 62) (width 0.2) (layer "B.Cu") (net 2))
 (segment (start 120.15 104) (end 129.5 104) (width 0.75) (layer "B.Cu") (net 2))
 (segment (start 179 90) (end 179 92) (width 0.2) (layer "B.Cu") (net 2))
 (segment (start 174.5 68) (end 178 68) (width 0.2) (layer "F.Cu") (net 11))
 (segment (start 178 68) (end 178 61.5) (width 0.2) (layer "F.Cu") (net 11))
 (segment (start 207.775 61.225) (end 212.275 61.225) (width 0.2) (layer "F.Cu") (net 11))
 (segment (start 168.275 67.775) (end 168.5 68) (width 0.2) (layer "F.Cu") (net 11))
 (segment (start 185.775 61.225) (end 191.275 61.225) (width 0.2) (layer "F.Cu") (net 11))
 (segment (start 168.5 68) (end 174.5 68) (width 0.2) (layer "F.Cu") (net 11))
 (segment (start 178 61.5) (end 178.2 61.3) (width 0.2) (layer "F.Cu") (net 11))
 (segment (start 202.275 61.225) (end 207.775 61.225) (width 0.2) (layer "F.Cu") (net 11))
 (segment (start 196.775 61.225) (end 202.275 61.225) (width 0.2) (layer "F.Cu") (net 11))
 (segment (start 178.2 61.3) (end 180.775 61.3) (width 0.2) (layer "F.Cu") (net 11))
 (segment (start 185.7 61.3) (end 185.775 61.225) (width 0.2) (layer "F.Cu") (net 11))
 (segment (start 180.775 61.3) (end 185.7 61.3) (width 0.2) (layer "F.Cu") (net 11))
 (segment (start 168.275 61.3) (end 168.275 67.775) (width 0.2) (layer "F.Cu") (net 11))
 (segment (start 191.275 61.225) (end 196.775 61.225) (width 0.2) (layer "F.Cu") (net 11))
 (segment (start 101.5 90.375) (end 101.5 98) (width 0.5) (layer "F.Cu") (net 1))
 (segment (start 122.5 87) (end 121.775 87.725) (width 0.5) (layer "F.Cu") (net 1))
 (segment (start 139 83.5) (end 139.265 83.765) (width 0.2) (layer "F.Cu") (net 1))
 (segment (start 101.5 98) (end 112.5 98) (width 0.5) (layer "F.Cu") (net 1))
 (segment (start 139.265 83.765) (end 139.265 87.775) (width 0.5) (layer "F.Cu") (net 1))
 (segment (start 121.775 61.8) (end 121.775 60.225) (width 0.5) (layer "F.Cu") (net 1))
 (segment (start 111.575 80.3) (end 101.5 90.375) (width 0.5) (layer "F.Cu") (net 1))
 (segment (start 111.575 80.3) (end 111.575 61.8) (width 0.5) (layer "F.Cu") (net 1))
 (segment (start 111.575 61.8) (end 121.775 61.8) (width 0.5) (layer "F.Cu") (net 1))
 (segment (start 121.775 60.225) (end 122 60) (width 0.2) (layer "F.Cu") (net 1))
 (segment (start 117.7 92.8) (end 121.775 92.8) (width 0.5) (layer "F.Cu") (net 1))
 (segment (start 112.5 98) (end 117.7 92.8) (width 0.5) (layer "F.Cu") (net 1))
 (segment (start 121.775 87.725) (end 121.775 92.8) (width 0.5) (layer "F.Cu") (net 1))
 (segment (start 139 58.5) (end 139.04 58.54) (width 0.2) (layer "F.Cu") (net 1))
 (segment (start 139.04 58.54) (end 139.04 62.225) (width 0.5) (layer "F.Cu") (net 1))
 (via (at 122 60) (size 1.2) (drill 0.6) (layers "F.Cu" "B.Cu") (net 1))
 (via (at 122.5 87) (size 1.2) (drill 0.6) (layers "F.Cu" "B.Cu") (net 1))
 (via (at 139 58.5) (size 1.2) (drill 0.6) (layers "F.Cu" "B.Cu") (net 1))
 (via (at 139 83.5) (size 1.2) (drill 0.6) (layers "F.Cu" "B.Cu") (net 1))
 (segment (start 122 60) (end 123.5 58.5) (width 0.5) (layer "B.Cu") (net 1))
 (segment (start 122.5 87) (end 122.5 86) (width 0.5) (layer "B.Cu") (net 1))
 (segment (start 122.5 86) (end 125 83.5) (width 0.5) (layer "B.Cu") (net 1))
 (segment (start 123.5 57.5) (end 139 57.5) (width 0.5) (layer "B.Cu") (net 1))
 (segment (start 123.5 58.5) (end 123.5 57.5) (width 0.5) (layer "B.Cu") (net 1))
 (segment (start 125 83.5) (end 139 83.5) (width 0.5) (layer "B.Cu") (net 1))
 (segment (start 139 57.5) (end 139 58.5) (width 0.5) (layer "B.Cu") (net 1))
 (segment (start 147.775 62.225) (end 148 62) (width 0.5) (layer "F.Cu") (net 3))
 (segment (start 156.775 61.3125) (end 165.4625 61.3125) (width 0.5) (layer "F.Cu") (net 3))
 (segment (start 148 61.0375) (end 156.5 61.0375) (width 0.5) (layer "F.Cu") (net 3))
 (segment (start 140.31 62.225) (end 147.775 62.225) (width 0.5) (layer "F.Cu") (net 3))
 (segment (start 156.725 61.2625) (end 156.775 61.3125) (width 0.2) (layer "F.Cu") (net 3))
 (segment (start 156.5 61.0375) (end 156.775 61.3125) (width 0.5) (layer "F.Cu") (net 3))
 (segment (start 148 62) (end 148 61.0375) (width 0.5) (layer "F.Cu") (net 3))
 (segment (start 165.4625 61.3125) (end 165.475 61.3) (width 0.2) (layer "F.Cu") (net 3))
 (segment (start 148 58.9625) (end 145.5375 56.5) (width 0.2) (layer "F.Cu") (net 4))
 (segment (start 137.77 56.73) (end 137.77 62.225) (width 0.2) (layer "F.Cu") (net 4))
 (segment (start 138 56.5) (end 137.77 56.73) (width 0.2) (layer "F.Cu") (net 4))
 (segment (start 145.5375 56.5) (end 138 56.5) (width 0.2) (layer "F.Cu") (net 4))
 (segment (start 137.77 64.525) (end 137.77 62.225) (width 0.2) (layer "F.Cu") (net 4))
 (segment (start 157.25 89.9625) (end 157.2875 90) (width 0.2) (layer "F.Cu") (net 9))
 (segment (start 147 90) (end 150 90) (width 0.5) (layer "F.Cu") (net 9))
 (segment (start 140.535 87.775) (end 144.775 87.775) (width 0.5) (layer "F.Cu") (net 9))
 (segment (start 144.775 87.775) (end 147 90) (width 0.5) (layer "F.Cu") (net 9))
 (segment (start 164.275 90) (end 164.475 89.8) (width 0.2) (layer "F.Cu") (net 9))
 (segment (start 150 90) (end 157.2875 90) (width 0.5) (layer "F.Cu") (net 9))
 (segment (start 157.2875 90) (end 164.275 90) (width 0.5) (layer "F.Cu") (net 9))
 (segment (start 150 87.925) (end 144.075 82) (width 0.2) (layer "F.Cu") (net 13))
 (segment (start 137.995 85.495) (end 137.995 87.775) (width 0.2) (layer "F.Cu") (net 13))
 (segment (start 136.5 84) (end 137.995 85.495) (width 0.2) (layer "F.Cu") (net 13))
 (segment (start 136.5 83.5) (end 136.5 84) (width 0.2) (layer "F.Cu") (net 13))
 (segment (start 144.075 82) (end 138 82) (width 0.2) (layer "F.Cu") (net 13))
 (segment (start 138 82) (end 136.5 83.5) (width 0.2) (layer "F.Cu") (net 13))
 (segment (start 137.995 90.075) (end 137.995 87.775) (width 0.2) (layer "F.Cu") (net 13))
 (segment (start 131.115 63.8) (end 132.69 62.225) (width 0.2) (layer "F.Cu") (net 7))
 (segment (start 121.775 63.8) (end 131.115 63.8) (width 0.2) (layer "F.Cu") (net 7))
 (segment (start 121.775 63.8) (end 121.775 70.3) (width 0.2) (layer "F.Cu") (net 7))
 (segment (start 121.775 94.8) (end 125.89 94.8) (width 0.2) (layer "F.Cu") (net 12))
 (segment (start 121.775 98) (end 121.775 94.8) (width 0.2) (layer "F.Cu") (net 12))
 (segment (start 125.89 94.8) (end 132.915 87.775) (width 0.2) (layer "F.Cu") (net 12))
 (segment (start 173.5 62) (end 169.5 58) (width 0.2) (layer "F.Cu") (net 6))
 (segment (start 133.96 55.54) (end 133.96 62.225) (width 0.2) (layer "F.Cu") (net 6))
 (segment (start 148.059744 55.5) (end 134 55.5) (width 0.2) (layer "F.Cu") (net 6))
 (segment (start 174.5 66) (end 174.5 62) (width 0.2) (layer "F.Cu") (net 6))
 (segment (start 169.5 58) (end 150.559744 58) (width 0.2) (layer "F.Cu") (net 6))
 (segment (start 134 55.5) (end 133.96 55.54) (width 0.2) (layer "F.Cu") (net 6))
 (segment (start 174.5 62) (end 173.5 62) (width 0.2) (layer "F.Cu") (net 6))
 (segment (start 133.96 62.225) (end 133.96 64.525) (width 0.2) (layer "F.Cu") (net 6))
 (segment (start 150.559744 58) (end 148.059744 55.5) (width 0.2) (layer "F.Cu") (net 6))
 (segment (start 154.022244 85.5) (end 149.522244 81) (width 0.2) (layer "F.Cu") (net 10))
 (segment (start 175.275 89.8) (end 175.275 85.5) (width 0.2) (layer "F.Cu") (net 10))
 (segment (start 134.185 83.315) (end 134.185 87.775) (width 0.2) (layer "F.Cu") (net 10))
 (segment (start 175.275 85.5) (end 154.022244 85.5) (width 0.2) (layer "F.Cu") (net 10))
 (segment (start 136.5 81) (end 134.185 83.315) (width 0.2) (layer "F.Cu") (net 10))
 (segment (start 149.522244 81) (end 136.5 81) (width 0.2) (layer "F.Cu") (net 10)))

